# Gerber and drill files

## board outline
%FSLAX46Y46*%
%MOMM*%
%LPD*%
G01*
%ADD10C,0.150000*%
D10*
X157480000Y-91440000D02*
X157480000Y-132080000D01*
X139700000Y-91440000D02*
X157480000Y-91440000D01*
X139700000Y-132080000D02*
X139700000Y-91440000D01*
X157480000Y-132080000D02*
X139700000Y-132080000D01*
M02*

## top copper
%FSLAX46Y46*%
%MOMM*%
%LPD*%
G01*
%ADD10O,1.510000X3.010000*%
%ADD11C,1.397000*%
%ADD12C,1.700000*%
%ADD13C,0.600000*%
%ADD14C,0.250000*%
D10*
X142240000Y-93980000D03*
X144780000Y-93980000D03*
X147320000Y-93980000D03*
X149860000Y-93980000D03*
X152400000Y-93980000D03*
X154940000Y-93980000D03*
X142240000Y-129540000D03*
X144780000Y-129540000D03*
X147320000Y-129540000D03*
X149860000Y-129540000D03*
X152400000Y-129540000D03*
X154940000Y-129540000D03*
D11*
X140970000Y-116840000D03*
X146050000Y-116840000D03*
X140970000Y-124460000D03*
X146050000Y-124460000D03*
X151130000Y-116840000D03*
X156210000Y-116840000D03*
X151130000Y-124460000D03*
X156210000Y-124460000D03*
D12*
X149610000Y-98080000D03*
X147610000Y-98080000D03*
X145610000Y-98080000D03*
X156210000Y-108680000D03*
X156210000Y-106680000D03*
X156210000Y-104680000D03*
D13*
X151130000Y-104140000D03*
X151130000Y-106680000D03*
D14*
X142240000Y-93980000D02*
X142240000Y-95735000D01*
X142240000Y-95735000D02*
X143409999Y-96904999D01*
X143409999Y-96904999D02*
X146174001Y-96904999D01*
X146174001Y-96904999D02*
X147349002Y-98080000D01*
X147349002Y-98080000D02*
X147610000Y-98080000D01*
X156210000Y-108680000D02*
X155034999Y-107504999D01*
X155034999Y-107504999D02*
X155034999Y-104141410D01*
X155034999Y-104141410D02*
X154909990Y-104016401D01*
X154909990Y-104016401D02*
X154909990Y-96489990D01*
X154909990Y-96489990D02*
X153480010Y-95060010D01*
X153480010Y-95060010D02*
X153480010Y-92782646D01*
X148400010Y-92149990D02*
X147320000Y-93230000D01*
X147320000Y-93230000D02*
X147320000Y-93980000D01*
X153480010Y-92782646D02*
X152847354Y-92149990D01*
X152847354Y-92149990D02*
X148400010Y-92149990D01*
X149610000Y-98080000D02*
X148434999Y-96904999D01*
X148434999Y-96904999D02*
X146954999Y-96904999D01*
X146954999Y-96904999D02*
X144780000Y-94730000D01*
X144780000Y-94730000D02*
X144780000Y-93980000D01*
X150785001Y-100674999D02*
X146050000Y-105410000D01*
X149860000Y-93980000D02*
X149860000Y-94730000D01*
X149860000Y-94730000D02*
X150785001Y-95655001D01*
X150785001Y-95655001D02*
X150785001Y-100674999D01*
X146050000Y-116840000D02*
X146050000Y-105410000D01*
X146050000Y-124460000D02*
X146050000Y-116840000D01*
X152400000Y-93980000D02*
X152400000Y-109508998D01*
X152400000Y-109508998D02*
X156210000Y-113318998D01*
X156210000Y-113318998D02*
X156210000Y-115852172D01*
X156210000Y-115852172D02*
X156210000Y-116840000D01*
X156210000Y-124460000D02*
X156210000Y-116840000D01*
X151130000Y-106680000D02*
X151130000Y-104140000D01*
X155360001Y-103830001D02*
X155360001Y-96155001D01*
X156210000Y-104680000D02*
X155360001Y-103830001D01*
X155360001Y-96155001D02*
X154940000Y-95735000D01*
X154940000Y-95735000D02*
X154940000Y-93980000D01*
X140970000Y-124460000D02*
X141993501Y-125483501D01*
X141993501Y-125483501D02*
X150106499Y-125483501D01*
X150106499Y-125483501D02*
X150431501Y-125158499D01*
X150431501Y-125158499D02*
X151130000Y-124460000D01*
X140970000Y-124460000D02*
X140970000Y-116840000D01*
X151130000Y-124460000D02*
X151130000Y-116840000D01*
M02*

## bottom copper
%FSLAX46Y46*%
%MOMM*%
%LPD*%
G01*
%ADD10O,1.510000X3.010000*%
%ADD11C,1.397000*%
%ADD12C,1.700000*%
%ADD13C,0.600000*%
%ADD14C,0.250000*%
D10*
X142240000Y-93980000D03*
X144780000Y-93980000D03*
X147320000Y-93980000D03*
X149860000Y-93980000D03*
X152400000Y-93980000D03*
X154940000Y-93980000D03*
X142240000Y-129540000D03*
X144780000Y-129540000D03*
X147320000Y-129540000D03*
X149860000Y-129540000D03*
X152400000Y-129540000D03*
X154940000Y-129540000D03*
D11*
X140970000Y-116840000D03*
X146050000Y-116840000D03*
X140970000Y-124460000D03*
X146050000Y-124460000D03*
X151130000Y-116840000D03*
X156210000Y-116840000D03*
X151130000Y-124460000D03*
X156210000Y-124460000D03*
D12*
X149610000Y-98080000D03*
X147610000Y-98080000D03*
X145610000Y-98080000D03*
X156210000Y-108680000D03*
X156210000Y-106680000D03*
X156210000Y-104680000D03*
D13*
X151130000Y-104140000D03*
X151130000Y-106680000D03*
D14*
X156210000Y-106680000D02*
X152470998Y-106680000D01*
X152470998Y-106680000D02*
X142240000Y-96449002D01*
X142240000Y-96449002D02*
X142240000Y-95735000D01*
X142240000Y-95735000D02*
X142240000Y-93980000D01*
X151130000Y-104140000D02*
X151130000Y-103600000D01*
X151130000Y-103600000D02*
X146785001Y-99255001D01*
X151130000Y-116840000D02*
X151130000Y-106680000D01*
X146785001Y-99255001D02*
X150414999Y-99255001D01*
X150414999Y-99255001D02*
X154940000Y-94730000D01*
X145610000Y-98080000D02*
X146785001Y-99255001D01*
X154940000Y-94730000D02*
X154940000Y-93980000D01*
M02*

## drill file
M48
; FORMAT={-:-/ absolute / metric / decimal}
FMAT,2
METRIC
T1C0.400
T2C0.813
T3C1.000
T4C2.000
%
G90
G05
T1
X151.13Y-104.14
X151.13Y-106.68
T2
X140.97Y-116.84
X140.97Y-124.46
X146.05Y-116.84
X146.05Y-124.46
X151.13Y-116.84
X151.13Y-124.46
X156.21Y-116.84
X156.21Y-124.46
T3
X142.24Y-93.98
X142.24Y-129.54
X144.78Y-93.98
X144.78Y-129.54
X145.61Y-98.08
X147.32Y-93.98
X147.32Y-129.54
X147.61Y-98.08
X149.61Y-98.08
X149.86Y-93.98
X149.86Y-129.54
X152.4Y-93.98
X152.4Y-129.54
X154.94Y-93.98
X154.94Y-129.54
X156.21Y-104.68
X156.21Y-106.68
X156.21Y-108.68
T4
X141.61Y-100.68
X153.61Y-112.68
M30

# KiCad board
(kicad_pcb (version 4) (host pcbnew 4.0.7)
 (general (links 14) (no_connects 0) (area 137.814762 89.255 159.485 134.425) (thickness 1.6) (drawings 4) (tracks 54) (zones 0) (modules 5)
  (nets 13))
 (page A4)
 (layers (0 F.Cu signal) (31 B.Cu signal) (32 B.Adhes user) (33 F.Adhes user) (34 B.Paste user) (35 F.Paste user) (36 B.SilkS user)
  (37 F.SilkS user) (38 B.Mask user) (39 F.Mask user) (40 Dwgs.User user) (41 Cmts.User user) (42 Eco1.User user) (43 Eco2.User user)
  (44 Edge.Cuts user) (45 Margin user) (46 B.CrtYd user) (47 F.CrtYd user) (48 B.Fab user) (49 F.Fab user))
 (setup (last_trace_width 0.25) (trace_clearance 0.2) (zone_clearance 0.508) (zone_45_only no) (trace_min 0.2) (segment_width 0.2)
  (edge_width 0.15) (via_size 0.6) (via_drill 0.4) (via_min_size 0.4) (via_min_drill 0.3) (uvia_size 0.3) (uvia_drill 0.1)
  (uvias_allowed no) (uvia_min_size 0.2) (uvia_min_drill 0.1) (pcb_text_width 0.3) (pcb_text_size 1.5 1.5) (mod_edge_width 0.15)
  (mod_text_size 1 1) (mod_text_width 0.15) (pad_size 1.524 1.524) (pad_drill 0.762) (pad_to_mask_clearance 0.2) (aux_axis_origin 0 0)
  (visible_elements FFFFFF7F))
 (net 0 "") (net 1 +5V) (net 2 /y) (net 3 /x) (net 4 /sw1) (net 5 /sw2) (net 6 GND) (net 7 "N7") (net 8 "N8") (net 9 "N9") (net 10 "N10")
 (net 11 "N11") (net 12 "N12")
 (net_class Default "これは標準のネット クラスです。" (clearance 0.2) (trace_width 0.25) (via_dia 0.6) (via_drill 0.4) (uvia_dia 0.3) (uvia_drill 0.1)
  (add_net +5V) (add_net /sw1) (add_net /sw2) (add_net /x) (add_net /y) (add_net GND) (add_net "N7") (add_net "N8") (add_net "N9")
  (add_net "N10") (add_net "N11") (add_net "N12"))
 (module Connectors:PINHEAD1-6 (layer F.Cu) (at 142.24 93.98)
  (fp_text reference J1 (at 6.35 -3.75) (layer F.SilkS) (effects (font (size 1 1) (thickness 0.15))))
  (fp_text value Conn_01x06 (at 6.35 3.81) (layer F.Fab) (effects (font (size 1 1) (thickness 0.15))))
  (pad 1 thru_hole oval (at 0 0) (size 1.51 3.01) (drill 1) (layers *.Cu *.Mask) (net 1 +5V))
  (pad 2 thru_hole oval (at 2.54 0) (size 1.51 3.01) (drill 1) (layers *.Cu *.Mask) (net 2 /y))
  (pad 3 thru_hole oval (at 5.08 0) (size 1.51 3.01) (drill 1) (layers *.Cu *.Mask) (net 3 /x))
  (pad 4 thru_hole oval (at 7.62 0) (size 1.51 3.01) (drill 1) (layers *.Cu *.Mask) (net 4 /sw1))
  (pad 5 thru_hole oval (at 10.16 0) (size 1.51 3.01) (drill 1) (layers *.Cu *.Mask) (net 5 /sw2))
  (pad 6 thru_hole oval (at 12.7 0) (size 1.51 3.01) (drill 1) (layers *.Cu *.Mask) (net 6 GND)))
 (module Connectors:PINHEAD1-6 (layer F.Cu) (at 142.24 129.54)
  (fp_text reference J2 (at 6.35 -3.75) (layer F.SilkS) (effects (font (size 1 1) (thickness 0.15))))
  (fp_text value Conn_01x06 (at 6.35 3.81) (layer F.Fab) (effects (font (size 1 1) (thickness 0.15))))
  (pad 1 thru_hole oval (at 0 0) (size 1.51 3.01) (drill 1) (layers *.Cu *.Mask) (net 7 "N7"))
  (pad 2 thru_hole oval (at 2.54 0) (size 1.51 3.01) (drill 1) (layers *.Cu *.Mask) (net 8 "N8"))
  (pad 3 thru_hole oval (at 5.08 0) (size 1.51 3.01) (drill 1) (layers *.Cu *.Mask) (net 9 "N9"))
  (pad 4 thru_hole oval (at 7.62 0) (size 1.51 3.01) (drill 1) (layers *.Cu *.Mask) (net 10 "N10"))
  (pad 5 thru_hole oval (at 10.16 0) (size 1.51 3.01) (drill 1) (layers *.Cu *.Mask) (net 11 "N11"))
  (pad 6 thru_hole oval (at 12.7 0) (size 1.51 3.01) (drill 1) (layers *.Cu *.Mask) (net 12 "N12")))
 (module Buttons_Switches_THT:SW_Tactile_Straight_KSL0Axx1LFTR (layer F.Cu) (at 140.97 124.46 90)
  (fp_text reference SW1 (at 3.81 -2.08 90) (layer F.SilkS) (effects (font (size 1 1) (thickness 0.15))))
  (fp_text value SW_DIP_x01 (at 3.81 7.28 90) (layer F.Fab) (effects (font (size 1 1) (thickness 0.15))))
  (pad 1 thru_hole circle (at 7.62 0 90) (size 1.397 1.397) (drill 0.8128) (layers *.Cu *.Mask) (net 6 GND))
  (pad 2 thru_hole circle (at 7.62 5.08 90) (size 1.397 1.397) (drill 0.8128) (layers *.Cu *.Mask) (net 4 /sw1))
  (pad 1 thru_hole circle (at 0 0 90) (size 1.397 1.397) (drill 0.8128) (layers *.Cu *.Mask) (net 6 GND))
  (pad 2 thru_hole circle (at 0 5.08 90) (size 1.397 1.397) (drill 0.8128) (layers *.Cu *.Mask) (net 4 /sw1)))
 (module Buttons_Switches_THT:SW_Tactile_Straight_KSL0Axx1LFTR (layer F.Cu) (at 151.13 124.46 90)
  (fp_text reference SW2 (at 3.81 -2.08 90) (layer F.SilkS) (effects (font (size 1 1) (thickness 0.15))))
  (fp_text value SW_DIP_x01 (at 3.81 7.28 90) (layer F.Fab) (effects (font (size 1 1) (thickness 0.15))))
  (pad 1 thru_hole circle (at 7.62 0 90) (size 1.397 1.397) (drill 0.8128) (layers *.Cu *.Mask) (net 6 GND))
  (pad 2 thru_hole circle (at 7.62 5.08 90) (size 1.397 1.397) (drill 0.8128) (layers *.Cu *.Mask) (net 5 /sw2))
  (pad 1 thru_hole circle (at 0 0 90) (size 1.397 1.397) (drill 0.8128) (layers *.Cu *.Mask) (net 6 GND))
  (pad 2 thru_hole circle (at 0 5.08 90) (size 1.397 1.397) (drill 0.8128) (layers *.Cu *.Mask) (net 5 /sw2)))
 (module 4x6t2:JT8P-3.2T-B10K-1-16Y (layer F.Cu) (at 147.61 106.68)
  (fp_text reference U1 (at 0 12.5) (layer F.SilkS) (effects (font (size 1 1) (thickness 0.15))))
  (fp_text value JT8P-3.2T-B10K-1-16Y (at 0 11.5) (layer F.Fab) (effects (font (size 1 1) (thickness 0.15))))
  (pad 1 thru_hole circle (at 2 -8.6) (size 1.7 1.7) (drill 1) (layers *.Cu *.Mask) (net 2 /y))
  (pad 2 thru_hole circle (at 0 -8.6) (size 1.7 1.7) (drill 1) (layers *.Cu *.Mask) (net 1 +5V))
  (pad 3 thru_hole circle (at -2 -8.6) (size 1.7 1.7) (drill 1) (layers *.Cu *.Mask) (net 6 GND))
  (pad 4 thru_hole circle (at 8.6 2) (size 1.7 1.7) (drill 1) (layers *.Cu *.Mask) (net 3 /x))
  (pad 5 thru_hole circle (at 8.6 0) (size 1.7 1.7) (drill 1) (layers *.Cu *.Mask) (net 1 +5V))
  (pad 6 thru_hole circle (at 8.6 -2) (size 1.7 1.7) (drill 1) (layers *.Cu *.Mask) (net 6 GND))
  (pad "" np_thru_hole circle (at 6 6) (size 2 2) (drill 2) (layers *.Cu *.Mask))
  (pad "" np_thru_hole circle (at -6 -6) (size 2 2) (drill 2) (layers *.Cu *.Mask)))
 (gr_line (start 157.48 91.44) (end 157.48 132.08) (layer Edge.Cuts) (width 0.15))
 (gr_line (start 139.7 91.44) (end 157.48 91.44) (layer Edge.Cuts) (width 0.15))
 (gr_line (start 139.7 132.08) (end 139.7 91.44) (layer Edge.Cuts) (width 0.15))
 (gr_line (start 157.48 132.08) (end 139.7 132.08) (layer Edge.Cuts) (width 0.15))
 (segment (start 142.24 93.98) (end 142.24 95.735) (width 0.25) (layer F.Cu) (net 1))
 (segment (start 142.24 95.735) (end 143.409999 96.904999) (width 0.25) (layer F.Cu) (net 1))
 (segment (start 143.409999 96.904999) (end 146.174001 96.904999) (width 0.25) (layer F.Cu) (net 1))
 (segment (start 146.174001 96.904999) (end 147.349002 98.08) (width 0.25) (layer F.Cu) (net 1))
 (segment (start 147.349002 98.08) (end 147.61 98.08) (width 0.25) (layer F.Cu) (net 1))
 (segment (start 156.21 106.68) (end 152.470998 106.68) (width 0.25) (layer B.Cu) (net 1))
 (segment (start 152.470998 106.68) (end 142.24 96.449002) (width 0.25) (layer B.Cu) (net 1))
 (segment (start 142.24 96.449002) (end 142.24 95.735) (width 0.25) (layer B.Cu) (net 1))
 (segment (start 142.24 95.735) (end 142.24 93.98) (width 0.25) (layer B.Cu) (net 1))
 (segment (start 156.21 108.68) (end 155.034999 107.504999) (width 0.25) (layer F.Cu) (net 3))
 (segment (start 155.034999 107.504999) (end 155.034999 104.14141) (width 0.25) (layer F.Cu) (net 3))
 (segment (start 155.034999 104.14141) (end 154.90999 104.016401) (width 0.25) (layer F.Cu) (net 3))
 (segment (start 154.90999 104.016401) (end 154.90999 96.48999) (width 0.25) (layer F.Cu) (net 3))
 (segment (start 154.90999 96.48999) (end 153.48001 95.06001) (width 0.25) (layer F.Cu) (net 3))
 (segment (start 153.48001 95.06001) (end 153.48001 92.782646) (width 0.25) (layer F.Cu) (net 3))
 (segment (start 148.40001 92.14999) (end 147.32 93.23) (width 0.25) (layer F.Cu) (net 3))
 (segment (start 147.32 93.23) (end 147.32 93.98) (width 0.25) (layer F.Cu) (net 3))
 (segment (start 153.48001 92.782646) (end 152.847354 92.14999) (width 0.25) (layer F.Cu) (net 3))
 (segment (start 152.847354 92.14999) (end 148.40001 92.14999) (width 0.25) (layer F.Cu) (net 3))
 (segment (start 149.61 98.08) (end 148.434999 96.904999) (width 0.25) (layer F.Cu) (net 2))
 (segment (start 148.434999 96.904999) (end 146.954999 96.904999) (width 0.25) (layer F.Cu) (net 2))
 (segment (start 146.954999 96.904999) (end 144.78 94.73) (width 0.25) (layer F.Cu) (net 2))
 (segment (start 144.78 94.73) (end 144.78 93.98) (width 0.25) (layer F.Cu) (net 2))
 (segment (start 150.785001 100.674999) (end 146.05 105.41) (width 0.25) (layer F.Cu) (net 4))
 (segment (start 149.86 93.98) (end 149.86 94.73) (width 0.25) (layer F.Cu) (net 4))
 (segment (start 149.86 94.73) (end 150.785001 95.655001) (width 0.25) (layer F.Cu) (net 4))
 (segment (start 150.785001 95.655001) (end 150.785001 100.674999) (width 0.25) (layer F.Cu) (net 4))
 (segment (start 146.05 116.84) (end 146.05 105.41) (width 0.25) (layer F.Cu) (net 4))
 (segment (start 146.05 124.46) (end 146.05 116.84) (width 0.25) (layer F.Cu) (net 4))
 (segment (start 152.4 93.98) (end 152.4 109.508998) (width 0.25) (layer F.Cu) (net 5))
 (segment (start 152.4 109.508998) (end 156.21 113.318998) (width 0.25) (layer F.Cu) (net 5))
 (segment (start 156.21 113.318998) (end 156.21 115.852172) (width 0.25) (layer F.Cu) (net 5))
 (segment (start 156.21 115.852172) (end 156.21 116.84) (width 0.25) (layer F.Cu) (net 5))
 (segment (start 156.21 124.46) (end 156.21 116.84) (width 0.25) (layer F.Cu) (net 5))
 (segment (start 151.13 104.14) (end 151.13 103.6) (width 0.25) (layer B.Cu) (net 6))
 (segment (start 151.13 103.6) (end 146.785001 99.255001) (width 0.25) (layer B.Cu) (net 6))
 (segment (start 151.13 106.68) (end 151.13 104.14) (width 0.25) (layer F.Cu) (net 6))
 (via (at 151.13 104.14) (size 0.6) (drill 0.4) (layers F.Cu B.Cu) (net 6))
 (via (at 151.13 106.68) (size 0.6) (drill 0.4) (layers F.Cu B.Cu) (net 6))
 (segment (start 151.13 116.84) (end 151.13 106.68) (width 0.25) (layer B.Cu) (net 6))
 (segment (start 146.785001 99.255001) (end 150.414999 99.255001) (width 0.25) (layer B.Cu) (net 6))
 (segment (start 150.414999 99.255001) (end 154.94 94.73) (width 0.25) (layer B.Cu) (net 6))
 (segment (start 145.61 98.08) (end 146.785001 99.255001) (width 0.25) (layer B.Cu) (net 6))
 (segment (start 154.94 94.73) (end 154.94 93.98) (width 0.25) (layer B.Cu) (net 6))
 (segment (start 155.360001 103.830001) (end 155.360001 96.155001) (width 0.25) (layer F.Cu) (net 6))
 (segment (start 156.21 104.68) (end 155.360001 103.830001) (width 0.25) (layer F.Cu) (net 6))
 (segment (start 155.360001 96.155001) (end 154.94 95.735) (width 0.25) (layer F.Cu) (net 6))
 (segment (start 154.94 95.735) (end 154.94 93.98) (width 0.25) (layer F.Cu) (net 6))
 (segment (start 140.97 124.46) (end 141.993501 125.483501) (width 0.25) (layer F.Cu) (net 6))
 (segment (start 141.993501 125.483501) (end 150.106499 125.483501) (width 0.25) (layer F.Cu) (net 6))
 (segment (start 150.106499 125.483501) (end 150.431501 125.158499) (width 0.25) (layer F.Cu) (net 6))
 (segment (start 150.431501 125.158499) (end 151.13 124.46) (width 0.25) (layer F.Cu) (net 6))
 (segment (start 140.97 124.46) (end 140.97 116.84) (width 0.25) (layer F.Cu) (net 6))
 (segment (start 151.13 124.46) (end 151.13 116.84) (width 0.25) (layer F.Cu) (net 6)))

